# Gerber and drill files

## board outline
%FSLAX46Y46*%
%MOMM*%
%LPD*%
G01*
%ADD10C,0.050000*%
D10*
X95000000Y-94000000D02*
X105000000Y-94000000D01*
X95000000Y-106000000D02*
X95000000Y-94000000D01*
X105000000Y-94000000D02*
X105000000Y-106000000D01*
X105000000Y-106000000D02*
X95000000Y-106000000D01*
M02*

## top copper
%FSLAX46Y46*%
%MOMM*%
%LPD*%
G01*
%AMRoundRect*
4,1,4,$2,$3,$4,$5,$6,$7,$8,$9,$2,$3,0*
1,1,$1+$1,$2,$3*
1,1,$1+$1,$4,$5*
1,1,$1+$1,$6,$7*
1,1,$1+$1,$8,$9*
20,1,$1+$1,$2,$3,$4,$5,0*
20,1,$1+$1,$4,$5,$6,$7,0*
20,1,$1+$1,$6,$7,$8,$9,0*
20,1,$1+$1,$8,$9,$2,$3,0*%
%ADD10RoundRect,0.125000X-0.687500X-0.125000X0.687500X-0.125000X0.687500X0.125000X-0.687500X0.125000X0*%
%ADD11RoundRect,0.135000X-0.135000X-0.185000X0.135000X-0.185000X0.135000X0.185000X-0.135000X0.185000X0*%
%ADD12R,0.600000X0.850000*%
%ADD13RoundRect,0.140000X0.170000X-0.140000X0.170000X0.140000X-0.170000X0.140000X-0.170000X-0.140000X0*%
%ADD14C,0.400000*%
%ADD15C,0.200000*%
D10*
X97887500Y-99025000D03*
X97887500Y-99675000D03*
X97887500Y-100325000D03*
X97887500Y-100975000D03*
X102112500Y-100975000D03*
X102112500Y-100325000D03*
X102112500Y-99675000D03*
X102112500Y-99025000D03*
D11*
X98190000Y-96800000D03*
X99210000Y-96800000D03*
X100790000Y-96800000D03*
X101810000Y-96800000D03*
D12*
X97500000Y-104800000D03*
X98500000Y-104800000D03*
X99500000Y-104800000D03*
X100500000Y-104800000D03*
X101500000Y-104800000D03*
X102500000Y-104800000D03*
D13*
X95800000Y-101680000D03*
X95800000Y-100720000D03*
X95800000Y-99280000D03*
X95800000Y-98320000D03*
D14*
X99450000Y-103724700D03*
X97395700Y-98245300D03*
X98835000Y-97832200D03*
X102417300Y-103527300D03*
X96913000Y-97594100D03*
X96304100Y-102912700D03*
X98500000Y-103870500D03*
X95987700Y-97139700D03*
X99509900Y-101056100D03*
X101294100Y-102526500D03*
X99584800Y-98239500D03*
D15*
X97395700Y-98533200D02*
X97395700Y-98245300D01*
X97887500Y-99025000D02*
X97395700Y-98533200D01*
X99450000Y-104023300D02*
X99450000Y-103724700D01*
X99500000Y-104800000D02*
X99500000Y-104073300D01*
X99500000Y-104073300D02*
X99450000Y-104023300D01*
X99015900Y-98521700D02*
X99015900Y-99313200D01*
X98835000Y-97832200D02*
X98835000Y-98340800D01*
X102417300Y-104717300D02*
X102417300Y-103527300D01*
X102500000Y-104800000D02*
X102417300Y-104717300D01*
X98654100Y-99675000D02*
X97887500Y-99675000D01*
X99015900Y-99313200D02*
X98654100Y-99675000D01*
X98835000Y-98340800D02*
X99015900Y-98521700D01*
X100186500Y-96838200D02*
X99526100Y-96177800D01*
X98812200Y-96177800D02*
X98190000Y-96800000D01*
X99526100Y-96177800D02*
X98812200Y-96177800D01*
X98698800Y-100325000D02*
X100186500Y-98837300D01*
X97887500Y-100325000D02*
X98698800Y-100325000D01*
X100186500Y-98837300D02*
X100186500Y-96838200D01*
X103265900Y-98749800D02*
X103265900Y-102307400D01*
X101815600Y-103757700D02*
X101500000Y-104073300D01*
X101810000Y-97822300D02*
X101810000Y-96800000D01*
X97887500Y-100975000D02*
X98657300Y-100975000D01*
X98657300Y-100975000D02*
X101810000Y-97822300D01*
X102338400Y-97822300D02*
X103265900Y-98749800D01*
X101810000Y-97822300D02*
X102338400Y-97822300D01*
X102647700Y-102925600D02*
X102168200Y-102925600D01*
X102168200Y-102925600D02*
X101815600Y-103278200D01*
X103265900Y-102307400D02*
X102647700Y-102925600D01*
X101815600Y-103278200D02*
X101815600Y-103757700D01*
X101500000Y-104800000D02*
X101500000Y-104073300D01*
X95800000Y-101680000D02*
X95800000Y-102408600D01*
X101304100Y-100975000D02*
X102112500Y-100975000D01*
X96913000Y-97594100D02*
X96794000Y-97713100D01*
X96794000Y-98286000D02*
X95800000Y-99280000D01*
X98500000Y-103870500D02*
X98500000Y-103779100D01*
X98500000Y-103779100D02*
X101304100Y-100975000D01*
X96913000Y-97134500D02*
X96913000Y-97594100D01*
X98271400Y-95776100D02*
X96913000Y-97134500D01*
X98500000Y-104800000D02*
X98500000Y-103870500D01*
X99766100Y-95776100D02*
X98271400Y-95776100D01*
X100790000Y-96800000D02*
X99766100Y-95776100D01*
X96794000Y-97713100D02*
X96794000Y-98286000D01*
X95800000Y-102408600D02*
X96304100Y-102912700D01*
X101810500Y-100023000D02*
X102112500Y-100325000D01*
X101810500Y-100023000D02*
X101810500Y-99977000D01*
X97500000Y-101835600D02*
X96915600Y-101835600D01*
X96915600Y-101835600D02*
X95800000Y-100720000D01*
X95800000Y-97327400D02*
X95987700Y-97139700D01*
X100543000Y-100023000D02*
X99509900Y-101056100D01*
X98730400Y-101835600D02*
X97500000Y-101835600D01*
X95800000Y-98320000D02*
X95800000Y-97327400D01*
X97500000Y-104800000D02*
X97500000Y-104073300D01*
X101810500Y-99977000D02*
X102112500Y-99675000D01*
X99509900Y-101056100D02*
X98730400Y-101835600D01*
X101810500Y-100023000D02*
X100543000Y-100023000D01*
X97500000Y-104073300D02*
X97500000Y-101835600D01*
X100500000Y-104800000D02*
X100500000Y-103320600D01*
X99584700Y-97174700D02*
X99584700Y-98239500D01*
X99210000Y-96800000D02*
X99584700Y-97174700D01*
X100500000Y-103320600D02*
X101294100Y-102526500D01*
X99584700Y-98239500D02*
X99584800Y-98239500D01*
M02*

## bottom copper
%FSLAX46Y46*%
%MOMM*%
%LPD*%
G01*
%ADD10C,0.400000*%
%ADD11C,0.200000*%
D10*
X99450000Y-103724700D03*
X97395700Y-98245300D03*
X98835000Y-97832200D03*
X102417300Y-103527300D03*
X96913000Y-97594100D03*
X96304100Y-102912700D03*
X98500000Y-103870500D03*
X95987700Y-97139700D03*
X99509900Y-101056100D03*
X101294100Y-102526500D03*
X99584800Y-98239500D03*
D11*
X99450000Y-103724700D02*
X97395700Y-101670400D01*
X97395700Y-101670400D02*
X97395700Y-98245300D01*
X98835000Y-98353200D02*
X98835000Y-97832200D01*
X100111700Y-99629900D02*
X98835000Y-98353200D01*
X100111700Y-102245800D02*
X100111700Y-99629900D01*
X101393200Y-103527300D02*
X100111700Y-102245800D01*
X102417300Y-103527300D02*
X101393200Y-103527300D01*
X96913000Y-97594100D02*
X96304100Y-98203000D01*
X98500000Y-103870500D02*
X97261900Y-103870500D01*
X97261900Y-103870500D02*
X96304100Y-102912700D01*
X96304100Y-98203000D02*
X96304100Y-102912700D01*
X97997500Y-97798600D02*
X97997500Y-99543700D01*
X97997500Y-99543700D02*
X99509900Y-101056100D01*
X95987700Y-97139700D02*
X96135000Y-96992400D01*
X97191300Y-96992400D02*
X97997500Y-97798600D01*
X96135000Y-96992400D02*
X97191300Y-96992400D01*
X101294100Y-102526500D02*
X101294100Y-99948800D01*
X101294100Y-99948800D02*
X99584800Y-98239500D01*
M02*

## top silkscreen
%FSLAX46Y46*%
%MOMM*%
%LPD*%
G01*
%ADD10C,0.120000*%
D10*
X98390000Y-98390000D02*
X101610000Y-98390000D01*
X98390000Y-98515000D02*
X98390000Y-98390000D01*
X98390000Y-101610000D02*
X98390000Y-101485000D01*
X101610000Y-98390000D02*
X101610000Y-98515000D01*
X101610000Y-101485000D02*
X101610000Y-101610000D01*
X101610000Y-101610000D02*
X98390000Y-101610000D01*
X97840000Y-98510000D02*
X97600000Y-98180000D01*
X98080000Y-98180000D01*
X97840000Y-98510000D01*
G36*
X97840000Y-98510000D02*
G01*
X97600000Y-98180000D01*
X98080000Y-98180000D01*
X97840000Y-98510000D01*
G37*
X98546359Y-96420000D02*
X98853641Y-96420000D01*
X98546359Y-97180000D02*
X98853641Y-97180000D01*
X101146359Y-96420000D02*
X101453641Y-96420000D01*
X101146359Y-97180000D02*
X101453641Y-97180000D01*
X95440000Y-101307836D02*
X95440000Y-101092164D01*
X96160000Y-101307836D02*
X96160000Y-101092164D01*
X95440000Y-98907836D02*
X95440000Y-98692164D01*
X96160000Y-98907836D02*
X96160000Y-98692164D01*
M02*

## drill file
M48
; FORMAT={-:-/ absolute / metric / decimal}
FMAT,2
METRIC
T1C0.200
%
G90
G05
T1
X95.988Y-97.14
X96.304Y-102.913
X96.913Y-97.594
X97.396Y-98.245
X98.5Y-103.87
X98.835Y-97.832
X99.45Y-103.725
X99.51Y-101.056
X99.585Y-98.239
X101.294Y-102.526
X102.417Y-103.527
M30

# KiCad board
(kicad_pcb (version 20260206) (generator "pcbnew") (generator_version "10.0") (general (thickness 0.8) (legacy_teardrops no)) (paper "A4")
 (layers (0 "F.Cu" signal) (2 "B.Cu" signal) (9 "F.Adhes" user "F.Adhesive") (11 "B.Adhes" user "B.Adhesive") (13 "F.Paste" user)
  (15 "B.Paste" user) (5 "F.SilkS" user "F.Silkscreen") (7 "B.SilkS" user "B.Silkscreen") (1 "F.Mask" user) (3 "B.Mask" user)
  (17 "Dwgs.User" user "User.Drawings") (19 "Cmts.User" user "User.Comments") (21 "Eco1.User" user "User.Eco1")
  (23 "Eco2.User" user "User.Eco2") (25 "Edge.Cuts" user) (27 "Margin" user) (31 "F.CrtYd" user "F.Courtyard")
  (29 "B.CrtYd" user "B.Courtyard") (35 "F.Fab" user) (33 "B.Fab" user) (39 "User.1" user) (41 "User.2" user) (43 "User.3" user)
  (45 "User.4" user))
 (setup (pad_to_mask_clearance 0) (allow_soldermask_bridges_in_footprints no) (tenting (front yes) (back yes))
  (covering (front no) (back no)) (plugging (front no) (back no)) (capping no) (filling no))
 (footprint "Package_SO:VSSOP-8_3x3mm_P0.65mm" (layer "F.Cu") (at 100 100)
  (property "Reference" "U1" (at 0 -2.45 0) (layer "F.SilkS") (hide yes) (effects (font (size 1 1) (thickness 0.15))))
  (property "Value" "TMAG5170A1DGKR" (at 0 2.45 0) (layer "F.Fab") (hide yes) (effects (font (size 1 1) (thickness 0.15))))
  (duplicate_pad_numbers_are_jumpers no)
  (fp_line (start -1.61 -1.61) (end 1.61 -1.61) (stroke (width 0.12) (type solid)) (layer "F.SilkS"))
  (fp_line (start -1.61 -1.485) (end -1.61 -1.61) (stroke (width 0.12) (type solid)) (layer "F.SilkS"))
  (fp_line (start -1.61 1.61) (end -1.61 1.485) (stroke (width 0.12) (type solid)) (layer "F.SilkS"))
  (fp_line (start 1.61 -1.61) (end 1.61 -1.485) (stroke (width 0.12) (type solid)) (layer "F.SilkS"))
  (fp_line (start 1.61 1.485) (end 1.61 1.61) (stroke (width 0.12) (type solid)) (layer "F.SilkS"))
  (fp_line (start 1.61 1.61) (end -1.61 1.61) (stroke (width 0.12) (type solid)) (layer "F.SilkS"))
  (fp_poly (pts (xy -2.16 -1.49) (xy -2.4 -1.82) (xy -1.92 -1.82)) (stroke (width 0.12) (type solid)) (fill yes) (layer "F.SilkS"))
  (pad "1" smd roundrect (at -2.1125 -0.975) (size 1.625 0.5) (layers "F.Cu" "F.Mask" "F.Paste") (roundrect_rratio 0.25) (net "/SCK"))
  (pad "2" smd roundrect (at -2.1125 -0.325) (size 1.625 0.5) (layers "F.Cu" "F.Mask" "F.Paste") (roundrect_rratio 0.25) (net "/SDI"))
  (pad "3" smd roundrect (at -2.1125 0.325) (size 1.625 0.5) (layers "F.Cu" "F.Mask" "F.Paste") (roundrect_rratio 0.25) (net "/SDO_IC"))
  (pad "4" smd roundrect (at -2.1125 0.975) (size 1.625 0.5) (layers "F.Cu" "F.Mask" "F.Paste") (roundrect_rratio 0.25) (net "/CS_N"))
  (pad "5" smd roundrect (at 2.1125 0.975) (size 1.625 0.5) (layers "F.Cu" "F.Mask" "F.Paste") (roundrect_rratio 0.25) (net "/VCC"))
  (pad "6" smd roundrect (at 2.1125 0.325) (size 1.625 0.5) (layers "F.Cu" "F.Mask" "F.Paste") (roundrect_rratio 0.25) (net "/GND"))
  (pad "7" smd roundrect (at 2.1125 -0.325) (size 1.625 0.5) (layers "F.Cu" "F.Mask" "F.Paste") (roundrect_rratio 0.25) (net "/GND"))
  (pad "8" smd roundrect (at 2.1125 -0.975) (size 1.625 0.5) (layers "F.Cu" "F.Mask" "F.Paste") (roundrect_rratio 0.25)
   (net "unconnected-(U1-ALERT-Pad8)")))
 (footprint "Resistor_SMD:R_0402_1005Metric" (layer "F.Cu") (at 98.7 96.8)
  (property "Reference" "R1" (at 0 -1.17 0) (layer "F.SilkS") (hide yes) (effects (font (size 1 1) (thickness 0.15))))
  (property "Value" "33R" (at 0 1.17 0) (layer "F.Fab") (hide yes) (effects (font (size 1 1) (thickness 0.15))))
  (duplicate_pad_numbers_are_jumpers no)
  (fp_line (start -0.153641 -0.38) (end 0.153641 -0.38) (stroke (width 0.12) (type solid)) (layer "F.SilkS"))
  (fp_line (start -0.153641 0.38) (end 0.153641 0.38) (stroke (width 0.12) (type solid)) (layer "F.SilkS"))
  (pad "1" smd roundrect (at -0.51 0) (size 0.54 0.64) (layers "F.Cu" "F.Mask" "F.Paste") (roundrect_rratio 0.25) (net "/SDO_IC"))
  (pad "2" smd roundrect (at 0.51 0) (size 0.54 0.64) (layers "F.Cu" "F.Mask" "F.Paste") (roundrect_rratio 0.25) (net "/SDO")))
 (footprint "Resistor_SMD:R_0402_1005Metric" (layer "F.Cu") (at 101.3 96.8)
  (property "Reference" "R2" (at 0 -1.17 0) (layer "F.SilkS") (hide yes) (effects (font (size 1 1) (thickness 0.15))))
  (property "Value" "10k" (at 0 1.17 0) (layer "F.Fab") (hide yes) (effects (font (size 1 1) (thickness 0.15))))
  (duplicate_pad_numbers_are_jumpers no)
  (fp_line (start -0.153641 -0.38) (end 0.153641 -0.38) (stroke (width 0.12) (type solid)) (layer "F.SilkS"))
  (fp_line (start -0.153641 0.38) (end 0.153641 0.38) (stroke (width 0.12) (type solid)) (layer "F.SilkS"))
  (pad "1" smd roundrect (at -0.51 0) (size 0.54 0.64) (layers "F.Cu" "F.Mask" "F.Paste") (roundrect_rratio 0.25) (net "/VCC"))
  (pad "2" smd roundrect (at 0.51 0) (size 0.54 0.64) (layers "F.Cu" "F.Mask" "F.Paste") (roundrect_rratio 0.25) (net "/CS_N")))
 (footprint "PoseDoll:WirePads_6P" (layer "F.Cu") (at 100 104.8)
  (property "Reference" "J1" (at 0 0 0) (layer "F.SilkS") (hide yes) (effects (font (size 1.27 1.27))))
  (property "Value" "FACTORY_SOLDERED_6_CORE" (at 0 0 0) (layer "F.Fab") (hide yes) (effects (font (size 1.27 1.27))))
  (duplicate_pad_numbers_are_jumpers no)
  (pad "1" smd rect (at -2.5 0) (size 0.6 0.85) (layers "F.Cu" "F.Mask") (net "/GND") (thermal_bridge_angle 45))
  (pad "2" smd rect (at -1.5 0) (size 0.6 0.85) (layers "F.Cu" "F.Mask") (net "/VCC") (thermal_bridge_angle 45))
  (pad "3" smd rect (at -0.5 0) (size 0.6 0.85) (layers "F.Cu" "F.Mask") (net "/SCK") (thermal_bridge_angle 45))
  (pad "4" smd rect (at 0.5 0) (size 0.6 0.85) (layers "F.Cu" "F.Mask") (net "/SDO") (thermal_bridge_angle 45))
  (pad "5" smd rect (at 1.5 0) (size 0.6 0.85) (layers "F.Cu" "F.Mask") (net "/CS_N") (thermal_bridge_angle 45))
  (pad "6" smd rect (at 2.5 0) (size 0.6 0.85) (layers "F.Cu" "F.Mask") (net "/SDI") (thermal_bridge_angle 45)))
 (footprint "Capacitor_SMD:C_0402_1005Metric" (layer "F.Cu") (at 95.8 101.2 90)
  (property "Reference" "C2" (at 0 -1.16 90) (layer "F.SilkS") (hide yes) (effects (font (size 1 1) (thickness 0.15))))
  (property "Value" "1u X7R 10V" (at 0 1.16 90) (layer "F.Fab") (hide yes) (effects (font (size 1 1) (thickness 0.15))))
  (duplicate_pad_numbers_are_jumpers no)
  (fp_line (start -0.107836 -0.36) (end 0.107836 -0.36) (stroke (width 0.12) (type solid)) (layer "F.SilkS"))
  (fp_line (start -0.107836 0.36) (end 0.107836 0.36) (stroke (width 0.12) (type solid)) (layer "F.SilkS"))
  (pad "1" smd roundrect (at -0.48 0 90) (size 0.56 0.62) (layers "F.Cu" "F.Mask" "F.Paste") (roundrect_rratio 0.25) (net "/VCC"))
  (pad "2" smd roundrect (at 0.48 0 90) (size 0.56 0.62) (layers "F.Cu" "F.Mask" "F.Paste") (roundrect_rratio 0.25) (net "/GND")))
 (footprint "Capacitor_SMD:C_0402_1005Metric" (layer "F.Cu") (at 95.8 98.8 90)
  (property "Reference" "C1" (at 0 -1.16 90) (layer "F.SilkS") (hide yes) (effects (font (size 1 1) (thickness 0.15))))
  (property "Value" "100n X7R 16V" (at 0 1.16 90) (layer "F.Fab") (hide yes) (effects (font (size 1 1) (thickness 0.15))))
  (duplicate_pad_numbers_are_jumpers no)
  (fp_line (start -0.107836 -0.36) (end 0.107836 -0.36) (stroke (width 0.12) (type solid)) (layer "F.SilkS"))
  (fp_line (start -0.107836 0.36) (end 0.107836 0.36) (stroke (width 0.12) (type solid)) (layer "F.SilkS"))
  (pad "1" smd roundrect (at -0.48 0 90) (size 0.56 0.62) (layers "F.Cu" "F.Mask" "F.Paste") (roundrect_rratio 0.25) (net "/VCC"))
  (pad "2" smd roundrect (at 0.48 0 90) (size 0.56 0.62) (layers "F.Cu" "F.Mask" "F.Paste") (roundrect_rratio 0.25) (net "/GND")))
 (gr_line (start 95 94) (end 105 94) (stroke (width 0.05) (type default)) (layer "Edge.Cuts"))
 (gr_line (start 95 106) (end 95 94) (stroke (width 0.05) (type default)) (layer "Edge.Cuts"))
 (gr_line (start 105 94) (end 105 106) (stroke (width 0.05) (type default)) (layer "Edge.Cuts"))
 (gr_line (start 105 106) (end 95 106) (stroke (width 0.05) (type default)) (layer "Edge.Cuts"))
 (segment (start 97.3957 98.5332) (end 97.3957 98.2453) (width 0.2) (layer "F.Cu") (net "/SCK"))
 (segment (start 97.8875 99.025) (end 97.3957 98.5332) (width 0.2) (layer "F.Cu") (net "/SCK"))
 (segment (start 99.45 104.0233) (end 99.45 103.7247) (width 0.2) (layer "F.Cu") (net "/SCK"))
 (segment (start 99.5 104.8) (end 99.5 104.0733) (width 0.2) (layer "F.Cu") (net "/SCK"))
 (segment (start 99.5 104.0733) (end 99.45 104.0233) (width 0.2) (layer "F.Cu") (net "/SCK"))
 (via (at 99.45 103.7247) (size 0.4) (drill 0.2) (layers "F.Cu" "B.Cu") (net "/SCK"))
 (via (at 97.3957 98.2453) (size 0.4) (drill 0.2) (layers "F.Cu" "B.Cu") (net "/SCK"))
 (segment (start 99.45 103.7247) (end 97.3957 101.6704) (width 0.2) (layer "B.Cu") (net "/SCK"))
 (segment (start 97.3957 101.6704) (end 97.3957 98.2453) (width 0.2) (layer "B.Cu") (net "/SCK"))
 (segment (start 99.0159 98.5217) (end 99.0159 99.3132) (width 0.2) (layer "F.Cu") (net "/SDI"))
 (segment (start 98.835 97.8322) (end 98.835 98.3408) (width 0.2) (layer "F.Cu") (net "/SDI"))
 (segment (start 102.4173 104.7173) (end 102.4173 103.5273) (width 0.2) (layer "F.Cu") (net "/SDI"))
 (segment (start 102.5 104.8) (end 102.4173 104.7173) (width 0.2) (layer "F.Cu") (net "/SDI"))
 (segment (start 98.6541 99.675) (end 97.8875 99.675) (width 0.2) (layer "F.Cu") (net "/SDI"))
 (segment (start 99.0159 99.3132) (end 98.6541 99.675) (width 0.2) (layer "F.Cu") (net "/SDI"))
 (segment (start 98.835 98.3408) (end 99.0159 98.5217) (width 0.2) (layer "F.Cu") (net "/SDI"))
 (via (at 98.835 97.8322) (size 0.4) (drill 0.2) (layers "F.Cu" "B.Cu") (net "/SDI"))
 (via (at 102.4173 103.5273) (size 0.4) (drill 0.2) (layers "F.Cu" "B.Cu") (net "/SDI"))
 (segment (start 98.835 98.3532) (end 98.835 97.8322) (width 0.2) (layer "B.Cu") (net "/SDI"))
 (segment (start 100.1117 99.6299) (end 98.835 98.3532) (width 0.2) (layer "B.Cu") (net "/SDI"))
 (segment (start 100.1117 102.2458) (end 100.1117 99.6299) (width 0.2) (layer "B.Cu") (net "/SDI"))
 (segment (start 101.3932 103.5273) (end 100.1117 102.2458) (width 0.2) (layer "B.Cu") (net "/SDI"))
 (segment (start 102.4173 103.5273) (end 101.3932 103.5273) (width 0.2) (layer "B.Cu") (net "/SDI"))
 (segment (start 100.1865 96.8382) (end 99.5261 96.1778) (width 0.2) (layer "F.Cu") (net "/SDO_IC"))
 (segment (start 98.8122 96.1778) (end 98.19 96.8) (width 0.2) (layer "F.Cu") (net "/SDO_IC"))
 (segment (start 99.5261 96.1778) (end 98.8122 96.1778) (width 0.2) (layer "F.Cu") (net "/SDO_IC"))
 (segment (start 98.6988 100.325) (end 100.1865 98.8373) (width 0.2) (layer "F.Cu") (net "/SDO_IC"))
 (segment (start 97.8875 100.325) (end 98.6988 100.325) (width 0.2) (layer "F.Cu") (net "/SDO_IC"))
 (segment (start 100.1865 98.8373) (end 100.1865 96.8382) (width 0.2) (layer "F.Cu") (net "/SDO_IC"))
 (segment (start 103.2659 98.7498) (end 103.2659 102.3074) (width 0.2) (layer "F.Cu") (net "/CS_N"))
 (segment (start 101.8156 103.7577) (end 101.5 104.0733) (width 0.2) (layer "F.Cu") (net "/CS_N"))
 (segment (start 101.81 97.8223) (end 101.81 96.8) (width 0.2) (layer "F.Cu") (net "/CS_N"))
 (segment (start 97.8875 100.975) (end 98.6573 100.975) (width 0.2) (layer "F.Cu") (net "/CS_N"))
 (segment (start 98.6573 100.975) (end 101.81 97.8223) (width 0.2) (layer "F.Cu") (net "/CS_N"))
 (segment (start 102.3384 97.8223) (end 103.2659 98.7498) (width 0.2) (layer "F.Cu") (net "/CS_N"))
 (segment (start 101.81 97.8223) (end 102.3384 97.8223) (width 0.2) (layer "F.Cu") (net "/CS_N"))
 (segment (start 102.6477 102.9256) (end 102.1682 102.9256) (width 0.2) (layer "F.Cu") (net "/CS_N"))
 (segment (start 102.1682 102.9256) (end 101.8156 103.2782) (width 0.2) (layer "F.Cu") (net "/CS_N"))
 (segment (start 103.2659 102.3074) (end 102.6477 102.9256) (width 0.2) (layer "F.Cu") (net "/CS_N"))
 (segment (start 101.8156 103.2782) (end 101.8156 103.7577) (width 0.2) (layer "F.Cu") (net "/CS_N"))
 (segment (start 101.5 104.8) (end 101.5 104.0733) (width 0.2) (layer "F.Cu") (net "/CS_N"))
 (segment (start 95.8 101.68) (end 95.8 102.4086) (width 0.2) (layer "F.Cu") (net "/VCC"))
 (segment (start 101.3041 100.975) (end 102.1125 100.975) (width 0.2) (layer "F.Cu") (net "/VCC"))
 (segment (start 96.913 97.5941) (end 96.794 97.7131) (width 0.2) (layer "F.Cu") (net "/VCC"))
 (segment (start 96.794 98.286) (end 95.8 99.28) (width 0.2) (layer "F.Cu") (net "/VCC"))
 (segment (start 98.5 103.8705) (end 98.5 103.7791) (width 0.2) (layer "F.Cu") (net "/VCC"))
 (segment (start 98.5 103.7791) (end 101.3041 100.975) (width 0.2) (layer "F.Cu") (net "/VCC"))
 (segment (start 96.913 97.1345) (end 96.913 97.5941) (width 0.2) (layer "F.Cu") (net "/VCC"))
 (segment (start 98.2714 95.7761) (end 96.913 97.1345) (width 0.2) (layer "F.Cu") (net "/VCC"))
 (segment (start 98.5 104.8) (end 98.5 103.8705) (width 0.2) (layer "F.Cu") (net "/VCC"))
 (segment (start 99.7661 95.7761) (end 98.2714 95.7761) (width 0.2) (layer "F.Cu") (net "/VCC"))
 (segment (start 100.79 96.8) (end 99.7661 95.7761) (width 0.2) (layer "F.Cu") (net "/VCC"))
 (segment (start 96.794 97.7131) (end 96.794 98.286) (width 0.2) (layer "F.Cu") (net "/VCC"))
 (segment (start 95.8 102.4086) (end 96.3041 102.9127) (width 0.2) (layer "F.Cu") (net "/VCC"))
 (via (at 96.913 97.5941) (size 0.4) (drill 0.2) (layers "F.Cu" "B.Cu") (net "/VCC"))
 (via (at 96.3041 102.9127) (size 0.4) (drill 0.2) (layers "F.Cu" "B.Cu") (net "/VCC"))
 (via (at 98.5 103.8705) (size 0.4) (drill 0.2) (layers "F.Cu" "B.Cu") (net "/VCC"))
 (segment (start 96.913 97.5941) (end 96.3041 98.203) (width 0.2) (layer "B.Cu") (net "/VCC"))
 (segment (start 98.5 103.8705) (end 97.2619 103.8705) (width 0.2) (layer "B.Cu") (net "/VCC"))
 (segment (start 97.2619 103.8705) (end 96.3041 102.9127) (width 0.2) (layer "B.Cu") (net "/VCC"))
 (segment (start 96.3041 98.203) (end 96.3041 102.9127) (width 0.2) (layer "B.Cu") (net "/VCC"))
 (segment (start 101.8105 100.023) (end 102.1125 100.325) (width 0.2) (layer "F.Cu") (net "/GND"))
 (segment (start 101.8105 100.023) (end 101.8105 99.977) (width 0.2) (layer "F.Cu") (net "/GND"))
 (segment (start 97.5 101.8356) (end 96.9156 101.8356) (width 0.2) (layer "F.Cu") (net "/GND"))
 (segment (start 96.9156 101.8356) (end 95.8 100.72) (width 0.2) (layer "F.Cu") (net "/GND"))
 (segment (start 95.8 97.3274) (end 95.9877 97.1397) (width 0.2) (layer "F.Cu") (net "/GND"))
 (segment (start 100.543 100.023) (end 99.5099 101.0561) (width 0.2) (layer "F.Cu") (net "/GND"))
 (segment (start 98.7304 101.8356) (end 97.5 101.8356) (width 0.2) (layer "F.Cu") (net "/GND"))
 (segment (start 95.8 98.32) (end 95.8 97.3274) (width 0.2) (layer "F.Cu") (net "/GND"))
 (segment (start 97.5 104.8) (end 97.5 104.0733) (width 0.2) (layer "F.Cu") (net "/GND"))
 (segment (start 101.8105 99.977) (end 102.1125 99.675) (width 0.2) (layer "F.Cu") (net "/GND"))
 (segment (start 99.5099 101.0561) (end 98.7304 101.8356) (width 0.2) (layer "F.Cu") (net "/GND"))
 (segment (start 101.8105 100.023) (end 100.543 100.023) (width 0.2) (layer "F.Cu") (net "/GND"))
 (segment (start 97.5 104.0733) (end 97.5 101.8356) (width 0.2) (layer "F.Cu") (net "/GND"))
 (via (at 95.9877 97.1397) (size 0.4) (drill 0.2) (layers "F.Cu" "B.Cu") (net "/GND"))
 (via (at 99.5099 101.0561) (size 0.4) (drill 0.2) (layers "F.Cu" "B.Cu") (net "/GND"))
 (segment (start 97.9975 97.7986) (end 97.9975 99.5437) (width 0.2) (layer "B.Cu") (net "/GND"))
 (segment (start 97.9975 99.5437) (end 99.5099 101.0561) (width 0.2) (layer "B.Cu") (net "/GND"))
 (segment (start 95.9877 97.1397) (end 96.135 96.9924) (width 0.2) (layer "B.Cu") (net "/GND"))
 (segment (start 97.1913 96.9924) (end 97.9975 97.7986) (width 0.2) (layer "B.Cu") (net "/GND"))
 (segment (start 96.135 96.9924) (end 97.1913 96.9924) (width 0.2) (layer "B.Cu") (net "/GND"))
 (segment (start 100.5 104.8) (end 100.5 103.3206) (width 0.2) (layer "F.Cu") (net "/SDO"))
 (segment (start 99.5847 97.1747) (end 99.5847 98.2395) (width 0.2) (layer "F.Cu") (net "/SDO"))
 (segment (start 99.21 96.8) (end 99.5847 97.1747) (width 0.2) (layer "F.Cu") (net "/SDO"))
 (segment (start 100.5 103.3206) (end 101.2941 102.5265) (width 0.2) (layer "F.Cu") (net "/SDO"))
 (segment (start 99.5847 98.2395) (end 99.5848 98.2395) (width 0.2) (layer "F.Cu") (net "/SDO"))
 (via (at 101.2941 102.5265) (size 0.4) (drill 0.2) (layers "F.Cu" "B.Cu") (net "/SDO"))
 (via (at 99.5848 98.2395) (size 0.4) (drill 0.2) (layers "F.Cu" "B.Cu") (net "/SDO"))
 (segment (start 101.2941 102.5265) (end 101.2941 99.9488) (width 0.2) (layer "B.Cu") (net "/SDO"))
 (segment (start 101.2941 99.9488) (end 99.5848 98.2395) (width 0.2) (layer "B.Cu") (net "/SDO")))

